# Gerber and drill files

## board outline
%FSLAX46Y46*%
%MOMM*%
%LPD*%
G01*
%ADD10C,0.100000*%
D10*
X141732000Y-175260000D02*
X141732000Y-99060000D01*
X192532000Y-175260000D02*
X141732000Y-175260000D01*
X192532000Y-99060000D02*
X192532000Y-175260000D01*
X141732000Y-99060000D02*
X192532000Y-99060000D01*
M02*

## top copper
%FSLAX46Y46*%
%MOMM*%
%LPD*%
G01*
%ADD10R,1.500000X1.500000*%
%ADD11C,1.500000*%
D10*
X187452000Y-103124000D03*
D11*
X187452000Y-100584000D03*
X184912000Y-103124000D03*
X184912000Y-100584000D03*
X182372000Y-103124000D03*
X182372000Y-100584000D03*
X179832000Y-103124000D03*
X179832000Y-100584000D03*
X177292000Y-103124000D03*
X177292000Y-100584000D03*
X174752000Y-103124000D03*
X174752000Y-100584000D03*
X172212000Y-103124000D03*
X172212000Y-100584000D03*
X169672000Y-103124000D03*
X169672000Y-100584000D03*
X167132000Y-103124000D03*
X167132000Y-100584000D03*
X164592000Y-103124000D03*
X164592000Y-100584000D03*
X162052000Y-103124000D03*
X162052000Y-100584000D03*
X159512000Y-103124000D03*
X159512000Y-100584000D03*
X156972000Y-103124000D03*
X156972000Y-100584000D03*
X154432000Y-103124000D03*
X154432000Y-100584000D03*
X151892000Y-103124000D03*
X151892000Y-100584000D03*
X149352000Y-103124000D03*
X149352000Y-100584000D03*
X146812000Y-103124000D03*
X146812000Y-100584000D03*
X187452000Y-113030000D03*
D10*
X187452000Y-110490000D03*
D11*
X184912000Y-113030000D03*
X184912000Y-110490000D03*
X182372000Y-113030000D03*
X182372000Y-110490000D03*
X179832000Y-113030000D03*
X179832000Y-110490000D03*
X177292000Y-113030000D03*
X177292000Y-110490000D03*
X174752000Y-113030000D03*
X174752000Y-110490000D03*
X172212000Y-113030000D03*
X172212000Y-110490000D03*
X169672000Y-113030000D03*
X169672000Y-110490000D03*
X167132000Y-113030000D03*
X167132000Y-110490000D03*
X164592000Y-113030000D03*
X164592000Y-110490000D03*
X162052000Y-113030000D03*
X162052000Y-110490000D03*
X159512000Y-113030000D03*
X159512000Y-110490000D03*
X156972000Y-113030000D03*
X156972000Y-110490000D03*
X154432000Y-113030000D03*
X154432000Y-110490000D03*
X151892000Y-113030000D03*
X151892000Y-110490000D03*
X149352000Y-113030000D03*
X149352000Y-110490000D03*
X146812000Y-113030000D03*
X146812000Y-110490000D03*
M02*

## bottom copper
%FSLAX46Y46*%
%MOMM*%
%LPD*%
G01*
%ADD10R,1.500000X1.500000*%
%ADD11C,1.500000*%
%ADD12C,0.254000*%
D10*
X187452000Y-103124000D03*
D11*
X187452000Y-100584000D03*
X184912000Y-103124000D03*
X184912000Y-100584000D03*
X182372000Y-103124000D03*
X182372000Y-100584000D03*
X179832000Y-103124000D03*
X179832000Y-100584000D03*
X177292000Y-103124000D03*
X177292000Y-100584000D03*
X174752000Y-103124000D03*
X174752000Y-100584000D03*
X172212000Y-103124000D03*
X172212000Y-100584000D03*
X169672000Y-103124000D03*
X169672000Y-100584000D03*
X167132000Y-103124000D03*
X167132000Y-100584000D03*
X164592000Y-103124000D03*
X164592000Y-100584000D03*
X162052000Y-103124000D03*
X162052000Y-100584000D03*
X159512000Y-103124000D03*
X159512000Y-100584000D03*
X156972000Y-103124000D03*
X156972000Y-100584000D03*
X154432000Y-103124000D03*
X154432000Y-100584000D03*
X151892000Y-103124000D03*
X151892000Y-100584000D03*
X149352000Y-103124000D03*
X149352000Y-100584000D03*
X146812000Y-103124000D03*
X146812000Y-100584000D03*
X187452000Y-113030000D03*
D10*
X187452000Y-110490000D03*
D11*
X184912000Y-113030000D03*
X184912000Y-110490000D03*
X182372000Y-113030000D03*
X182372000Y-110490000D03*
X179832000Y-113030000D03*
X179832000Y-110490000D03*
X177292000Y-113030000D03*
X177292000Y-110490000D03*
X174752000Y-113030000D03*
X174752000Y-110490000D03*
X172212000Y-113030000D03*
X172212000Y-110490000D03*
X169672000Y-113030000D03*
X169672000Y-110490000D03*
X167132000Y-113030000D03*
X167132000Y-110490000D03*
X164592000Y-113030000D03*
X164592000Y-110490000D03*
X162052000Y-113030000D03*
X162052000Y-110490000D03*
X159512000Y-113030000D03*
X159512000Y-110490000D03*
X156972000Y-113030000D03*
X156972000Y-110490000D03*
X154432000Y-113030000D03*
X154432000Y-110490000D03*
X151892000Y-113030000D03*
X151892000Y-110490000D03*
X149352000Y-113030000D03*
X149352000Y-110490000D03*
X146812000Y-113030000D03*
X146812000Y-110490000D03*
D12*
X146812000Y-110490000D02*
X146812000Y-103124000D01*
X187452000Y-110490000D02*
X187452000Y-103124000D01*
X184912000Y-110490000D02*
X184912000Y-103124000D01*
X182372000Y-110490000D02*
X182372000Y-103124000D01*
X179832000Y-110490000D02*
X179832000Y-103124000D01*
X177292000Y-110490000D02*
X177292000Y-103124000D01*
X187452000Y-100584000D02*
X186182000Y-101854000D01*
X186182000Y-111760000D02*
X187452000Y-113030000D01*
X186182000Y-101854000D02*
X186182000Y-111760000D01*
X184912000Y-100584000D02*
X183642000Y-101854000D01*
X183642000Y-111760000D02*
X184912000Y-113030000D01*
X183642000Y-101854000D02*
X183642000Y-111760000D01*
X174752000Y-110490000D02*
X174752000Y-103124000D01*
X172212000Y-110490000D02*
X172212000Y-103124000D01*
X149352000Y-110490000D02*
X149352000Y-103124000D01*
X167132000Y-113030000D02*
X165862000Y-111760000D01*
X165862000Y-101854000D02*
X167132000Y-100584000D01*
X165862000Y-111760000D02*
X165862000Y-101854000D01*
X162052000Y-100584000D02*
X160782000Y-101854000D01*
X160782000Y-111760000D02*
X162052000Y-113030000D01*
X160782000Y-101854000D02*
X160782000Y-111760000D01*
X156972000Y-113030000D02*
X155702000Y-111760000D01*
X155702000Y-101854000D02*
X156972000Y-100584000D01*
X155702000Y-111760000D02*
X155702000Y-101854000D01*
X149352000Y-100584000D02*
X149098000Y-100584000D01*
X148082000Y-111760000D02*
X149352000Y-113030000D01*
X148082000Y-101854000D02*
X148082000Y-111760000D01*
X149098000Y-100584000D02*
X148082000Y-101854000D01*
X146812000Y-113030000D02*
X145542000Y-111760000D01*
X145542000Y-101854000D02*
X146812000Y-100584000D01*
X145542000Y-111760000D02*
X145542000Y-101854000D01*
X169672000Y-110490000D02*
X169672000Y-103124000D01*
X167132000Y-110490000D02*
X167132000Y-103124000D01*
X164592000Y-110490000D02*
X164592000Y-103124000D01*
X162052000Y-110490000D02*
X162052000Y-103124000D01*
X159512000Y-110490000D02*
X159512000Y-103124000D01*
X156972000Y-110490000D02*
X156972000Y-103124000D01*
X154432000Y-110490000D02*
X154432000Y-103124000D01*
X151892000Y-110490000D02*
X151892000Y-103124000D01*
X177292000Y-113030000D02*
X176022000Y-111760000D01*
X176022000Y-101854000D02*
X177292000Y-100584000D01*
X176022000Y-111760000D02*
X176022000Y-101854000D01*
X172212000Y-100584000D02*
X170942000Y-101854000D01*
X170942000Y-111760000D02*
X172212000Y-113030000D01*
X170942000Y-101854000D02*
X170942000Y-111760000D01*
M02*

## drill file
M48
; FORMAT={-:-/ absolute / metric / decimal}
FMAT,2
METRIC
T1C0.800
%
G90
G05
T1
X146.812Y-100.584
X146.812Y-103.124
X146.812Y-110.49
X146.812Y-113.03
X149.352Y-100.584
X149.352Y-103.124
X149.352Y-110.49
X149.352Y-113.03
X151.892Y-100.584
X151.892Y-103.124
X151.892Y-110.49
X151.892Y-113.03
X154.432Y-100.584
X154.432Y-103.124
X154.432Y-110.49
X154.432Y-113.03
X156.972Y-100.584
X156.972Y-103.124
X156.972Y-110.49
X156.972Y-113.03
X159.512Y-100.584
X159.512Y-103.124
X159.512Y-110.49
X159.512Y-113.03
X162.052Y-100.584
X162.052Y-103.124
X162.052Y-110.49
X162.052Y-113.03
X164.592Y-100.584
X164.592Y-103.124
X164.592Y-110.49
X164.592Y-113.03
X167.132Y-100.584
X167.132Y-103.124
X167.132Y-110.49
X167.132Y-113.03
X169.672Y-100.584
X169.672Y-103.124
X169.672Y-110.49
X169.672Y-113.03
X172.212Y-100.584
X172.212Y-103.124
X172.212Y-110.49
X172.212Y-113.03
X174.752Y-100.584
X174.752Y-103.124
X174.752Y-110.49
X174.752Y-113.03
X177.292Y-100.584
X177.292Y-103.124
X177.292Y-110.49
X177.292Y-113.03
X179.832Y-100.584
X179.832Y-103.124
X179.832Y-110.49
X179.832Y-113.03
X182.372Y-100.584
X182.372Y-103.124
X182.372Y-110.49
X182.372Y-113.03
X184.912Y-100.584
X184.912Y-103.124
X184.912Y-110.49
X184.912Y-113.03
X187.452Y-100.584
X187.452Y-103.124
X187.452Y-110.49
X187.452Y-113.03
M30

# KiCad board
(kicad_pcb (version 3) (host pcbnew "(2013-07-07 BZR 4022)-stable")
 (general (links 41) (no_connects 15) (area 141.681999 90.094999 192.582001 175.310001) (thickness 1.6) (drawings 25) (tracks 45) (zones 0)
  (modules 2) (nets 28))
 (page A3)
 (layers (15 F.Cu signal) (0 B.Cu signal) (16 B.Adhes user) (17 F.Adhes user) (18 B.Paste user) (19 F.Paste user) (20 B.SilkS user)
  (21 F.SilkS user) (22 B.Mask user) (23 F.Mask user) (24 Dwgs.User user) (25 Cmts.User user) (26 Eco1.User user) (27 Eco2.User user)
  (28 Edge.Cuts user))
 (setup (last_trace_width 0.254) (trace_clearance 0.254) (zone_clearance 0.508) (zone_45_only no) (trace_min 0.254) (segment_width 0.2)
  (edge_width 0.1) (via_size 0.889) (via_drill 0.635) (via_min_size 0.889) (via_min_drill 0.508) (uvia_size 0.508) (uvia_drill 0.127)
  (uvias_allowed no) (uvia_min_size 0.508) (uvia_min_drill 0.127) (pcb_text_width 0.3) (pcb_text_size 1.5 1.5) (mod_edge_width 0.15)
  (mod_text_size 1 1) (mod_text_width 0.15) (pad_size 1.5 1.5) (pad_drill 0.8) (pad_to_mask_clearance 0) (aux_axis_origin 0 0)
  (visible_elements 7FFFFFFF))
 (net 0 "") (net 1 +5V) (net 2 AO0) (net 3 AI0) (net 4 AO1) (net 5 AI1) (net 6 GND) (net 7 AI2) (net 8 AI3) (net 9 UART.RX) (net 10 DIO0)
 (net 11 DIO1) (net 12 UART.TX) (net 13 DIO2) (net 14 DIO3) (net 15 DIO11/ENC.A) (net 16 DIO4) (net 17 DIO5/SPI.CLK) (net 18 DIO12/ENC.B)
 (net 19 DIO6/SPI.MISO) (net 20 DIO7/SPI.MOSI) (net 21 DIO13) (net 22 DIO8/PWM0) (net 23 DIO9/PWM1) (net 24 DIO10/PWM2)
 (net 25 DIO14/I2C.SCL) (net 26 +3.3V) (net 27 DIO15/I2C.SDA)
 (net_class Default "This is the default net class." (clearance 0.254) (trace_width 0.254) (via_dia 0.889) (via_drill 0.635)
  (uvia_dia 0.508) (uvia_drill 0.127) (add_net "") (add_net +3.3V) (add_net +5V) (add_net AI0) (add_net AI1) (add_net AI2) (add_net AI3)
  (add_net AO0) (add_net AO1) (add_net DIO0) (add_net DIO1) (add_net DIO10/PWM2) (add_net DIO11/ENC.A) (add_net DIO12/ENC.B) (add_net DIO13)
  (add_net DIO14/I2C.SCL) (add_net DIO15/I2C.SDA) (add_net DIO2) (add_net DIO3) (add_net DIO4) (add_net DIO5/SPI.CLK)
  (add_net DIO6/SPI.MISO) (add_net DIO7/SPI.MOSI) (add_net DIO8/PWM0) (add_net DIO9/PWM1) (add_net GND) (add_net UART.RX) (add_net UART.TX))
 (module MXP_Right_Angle (layer F.Cu) (at 168.402 101.854)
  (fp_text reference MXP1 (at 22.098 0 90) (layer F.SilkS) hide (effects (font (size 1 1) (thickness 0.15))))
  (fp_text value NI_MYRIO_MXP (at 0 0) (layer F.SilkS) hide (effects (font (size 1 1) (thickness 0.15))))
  (pad 1 thru_hole rect (at 19.05 1.27) (size 1.5 1.5) (drill 0.8) (layers *.Cu *.Mask F.SilkS) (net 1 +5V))
  (pad 2 thru_hole circle (at 19.05 -1.27) (size 1.5 1.5) (drill 0.8) (layers *.Cu *.Mask F.SilkS) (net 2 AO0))
  (pad 3 thru_hole circle (at 16.51 1.27) (size 1.5 1.5) (drill 0.8) (layers *.Cu *.Mask F.SilkS) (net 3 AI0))
  (pad 4 thru_hole circle (at 16.51 -1.27) (size 1.5 1.5) (drill 0.8) (layers *.Cu *.Mask F.SilkS) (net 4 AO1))
  (pad 5 thru_hole circle (at 13.97 1.27) (size 1.5 1.5) (drill 0.8) (layers *.Cu *.Mask F.SilkS) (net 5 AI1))
  (pad 6 thru_hole circle (at 13.97 -1.27) (size 1.5 1.5) (drill 0.8) (layers *.Cu *.Mask F.SilkS) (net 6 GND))
  (pad 7 thru_hole circle (at 11.43 1.27) (size 1.5 1.5) (drill 0.8) (layers *.Cu *.Mask F.SilkS) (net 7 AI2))
  (pad 8 thru_hole circle (at 11.43 -1.27) (size 1.5 1.5) (drill 0.8) (layers *.Cu *.Mask F.SilkS) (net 6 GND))
  (pad 9 thru_hole circle (at 8.89 1.27) (size 1.5 1.5) (drill 0.8) (layers *.Cu *.Mask F.SilkS) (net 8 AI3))
  (pad 10 thru_hole circle (at 8.89 -1.27) (size 1.5 1.5) (drill 0.8) (layers *.Cu *.Mask F.SilkS) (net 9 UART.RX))
  (pad 11 thru_hole circle (at 6.35 1.27) (size 1.5 1.5) (drill 0.8) (layers *.Cu *.Mask F.SilkS) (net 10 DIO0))
  (pad 12 thru_hole circle (at 6.35 -1.27) (size 1.5 1.5) (drill 0.8) (layers *.Cu *.Mask F.SilkS) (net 6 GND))
  (pad 13 thru_hole circle (at 3.81 1.27) (size 1.5 1.5) (drill 0.8) (layers *.Cu *.Mask F.SilkS) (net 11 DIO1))
  (pad 14 thru_hole circle (at 3.81 -1.27) (size 1.5 1.5) (drill 0.8) (layers *.Cu *.Mask F.SilkS) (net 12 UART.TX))
  (pad 15 thru_hole circle (at 1.27 1.27) (size 1.5 1.5) (drill 0.8) (layers *.Cu *.Mask F.SilkS) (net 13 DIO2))
  (pad 16 thru_hole circle (at 1.27 -1.27) (size 1.5 1.5) (drill 0.8) (layers *.Cu *.Mask F.SilkS) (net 6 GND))
  (pad 17 thru_hole circle (at -1.27 1.27) (size 1.5 1.5) (drill 0.8) (layers *.Cu *.Mask F.SilkS) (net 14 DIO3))
  (pad 18 thru_hole circle (at -1.27 -1.27) (size 1.5 1.5) (drill 0.8) (layers *.Cu *.Mask F.SilkS) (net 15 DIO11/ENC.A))
  (pad 19 thru_hole circle (at -3.81 1.27) (size 1.5 1.5) (drill 0.8) (layers *.Cu *.Mask F.SilkS) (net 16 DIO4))
  (pad 20 thru_hole circle (at -3.81 -1.27) (size 1.5 1.5) (drill 0.8) (layers *.Cu *.Mask F.SilkS) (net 6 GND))
  (pad 21 thru_hole circle (at -6.35 1.27) (size 1.5 1.5) (drill 0.8) (layers *.Cu *.Mask F.SilkS) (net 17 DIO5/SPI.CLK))
  (pad 22 thru_hole circle (at -6.35 -1.27) (size 1.5 1.5) (drill 0.8) (layers *.Cu *.Mask F.SilkS) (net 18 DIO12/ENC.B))
  (pad 23 thru_hole circle (at -8.89 1.27) (size 1.5 1.5) (drill 0.8) (layers *.Cu *.Mask F.SilkS) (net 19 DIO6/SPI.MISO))
  (pad 24 thru_hole circle (at -8.89 -1.27) (size 1.5 1.5) (drill 0.8) (layers *.Cu *.Mask F.SilkS) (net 6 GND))
  (pad 25 thru_hole circle (at -11.43 1.27) (size 1.5 1.5) (drill 0.8) (layers *.Cu *.Mask F.SilkS) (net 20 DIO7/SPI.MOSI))
  (pad 26 thru_hole circle (at -11.43 -1.27) (size 1.5 1.5) (drill 0.8) (layers *.Cu *.Mask F.SilkS) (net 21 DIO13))
  (pad 27 thru_hole circle (at -13.97 1.27) (size 1.5 1.5) (drill 0.8) (layers *.Cu *.Mask F.SilkS) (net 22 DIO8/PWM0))
  (pad 28 thru_hole circle (at -13.97 -1.27) (size 1.5 1.5) (drill 0.8) (layers *.Cu *.Mask F.SilkS) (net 6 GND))
  (pad 29 thru_hole circle (at -16.51 1.27) (size 1.5 1.5) (drill 0.8) (layers *.Cu *.Mask F.SilkS) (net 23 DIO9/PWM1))
  (pad 30 thru_hole circle (at -16.51 -1.27) (size 1.5 1.5) (drill 0.8) (layers *.Cu *.Mask F.SilkS) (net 6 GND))
  (pad 31 thru_hole circle (at -19.05 1.27) (size 1.5 1.5) (drill 0.8) (layers *.Cu *.Mask F.SilkS) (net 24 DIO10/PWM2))
  (pad 32 thru_hole circle (at -19.05 -1.27) (size 1.5 1.5) (drill 0.8) (layers *.Cu *.Mask F.SilkS) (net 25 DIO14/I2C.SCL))
  (pad 33 thru_hole circle (at -21.59 1.27) (size 1.5 1.5) (drill 0.8) (layers *.Cu *.Mask F.SilkS) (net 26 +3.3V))
  (pad 34 thru_hole circle (at -21.59 -1.27) (size 1.5 1.5) (drill 0.8) (layers *.Cu *.Mask F.SilkS) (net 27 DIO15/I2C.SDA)))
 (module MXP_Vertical (layer F.Cu) (at 168.402 111.76)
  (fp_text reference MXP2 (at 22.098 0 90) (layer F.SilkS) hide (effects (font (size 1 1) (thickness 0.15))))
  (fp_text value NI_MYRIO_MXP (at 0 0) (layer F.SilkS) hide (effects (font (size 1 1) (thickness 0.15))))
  (pad 2 thru_hole circle (at 19.05 1.27) (size 1.5 1.5) (drill 0.8) (layers *.Cu *.Mask F.SilkS) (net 2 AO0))
  (pad 1 thru_hole rect (at 19.05 -1.27) (size 1.5 1.5) (drill 0.8) (layers *.Cu *.Mask F.SilkS) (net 1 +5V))
  (pad 4 thru_hole circle (at 16.51 1.27) (size 1.5 1.5) (drill 0.8) (layers *.Cu *.Mask F.SilkS) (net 4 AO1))
  (pad 3 thru_hole circle (at 16.51 -1.27) (size 1.5 1.5) (drill 0.8) (layers *.Cu *.Mask F.SilkS) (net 3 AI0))
  (pad 6 thru_hole circle (at 13.97 1.27) (size 1.5 1.5) (drill 0.8) (layers *.Cu *.Mask F.SilkS) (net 6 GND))
  (pad 5 thru_hole circle (at 13.97 -1.27) (size 1.5 1.5) (drill 0.8) (layers *.Cu *.Mask F.SilkS) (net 5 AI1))
  (pad 8 thru_hole circle (at 11.43 1.27) (size 1.5 1.5) (drill 0.8) (layers *.Cu *.Mask F.SilkS) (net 6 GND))
  (pad 7 thru_hole circle (at 11.43 -1.27) (size 1.5 1.5) (drill 0.8) (layers *.Cu *.Mask F.SilkS) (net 7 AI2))
  (pad 10 thru_hole circle (at 8.89 1.27) (size 1.5 1.5) (drill 0.8) (layers *.Cu *.Mask F.SilkS) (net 9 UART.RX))
  (pad 9 thru_hole circle (at 8.89 -1.27) (size 1.5 1.5) (drill 0.8) (layers *.Cu *.Mask F.SilkS) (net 8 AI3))
  (pad 12 thru_hole circle (at 6.35 1.27) (size 1.5 1.5) (drill 0.8) (layers *.Cu *.Mask F.SilkS) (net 6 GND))
  (pad 11 thru_hole circle (at 6.35 -1.27) (size 1.5 1.5) (drill 0.8) (layers *.Cu *.Mask F.SilkS) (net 10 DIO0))
  (pad 14 thru_hole circle (at 3.81 1.27) (size 1.5 1.5) (drill 0.8) (layers *.Cu *.Mask F.SilkS) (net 12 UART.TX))
  (pad 13 thru_hole circle (at 3.81 -1.27) (size 1.5 1.5) (drill 0.8) (layers *.Cu *.Mask F.SilkS) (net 11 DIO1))
  (pad 16 thru_hole circle (at 1.27 1.27) (size 1.5 1.5) (drill 0.8) (layers *.Cu *.Mask F.SilkS) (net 6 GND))
  (pad 15 thru_hole circle (at 1.27 -1.27) (size 1.5 1.5) (drill 0.8) (layers *.Cu *.Mask F.SilkS) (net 13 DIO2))
  (pad 18 thru_hole circle (at -1.27 1.27) (size 1.5 1.5) (drill 0.8) (layers *.Cu *.Mask F.SilkS) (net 15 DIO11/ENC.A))
  (pad 17 thru_hole circle (at -1.27 -1.27) (size 1.5 1.5) (drill 0.8) (layers *.Cu *.Mask F.SilkS) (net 14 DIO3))
  (pad 20 thru_hole circle (at -3.81 1.27) (size 1.5 1.5) (drill 0.8) (layers *.Cu *.Mask F.SilkS) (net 6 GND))
  (pad 19 thru_hole circle (at -3.81 -1.27) (size 1.5 1.5) (drill 0.8) (layers *.Cu *.Mask F.SilkS) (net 16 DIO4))
  (pad 22 thru_hole circle (at -6.35 1.27) (size 1.5 1.5) (drill 0.8) (layers *.Cu *.Mask F.SilkS) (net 18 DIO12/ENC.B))
  (pad 21 thru_hole circle (at -6.35 -1.27) (size 1.5 1.5) (drill 0.8) (layers *.Cu *.Mask F.SilkS) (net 17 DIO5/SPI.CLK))
  (pad 24 thru_hole circle (at -8.89 1.27) (size 1.5 1.5) (drill 0.8) (layers *.Cu *.Mask F.SilkS) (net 6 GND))
  (pad 23 thru_hole circle (at -8.89 -1.27) (size 1.5 1.5) (drill 0.8) (layers *.Cu *.Mask F.SilkS) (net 19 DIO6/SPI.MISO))
  (pad 26 thru_hole circle (at -11.43 1.27) (size 1.5 1.5) (drill 0.8) (layers *.Cu *.Mask F.SilkS) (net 21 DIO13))
  (pad 25 thru_hole circle (at -11.43 -1.27) (size 1.5 1.5) (drill 0.8) (layers *.Cu *.Mask F.SilkS) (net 20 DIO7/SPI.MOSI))
  (pad 28 thru_hole circle (at -13.97 1.27) (size 1.5 1.5) (drill 0.8) (layers *.Cu *.Mask F.SilkS) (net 6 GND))
  (pad 27 thru_hole circle (at -13.97 -1.27) (size 1.5 1.5) (drill 0.8) (layers *.Cu *.Mask F.SilkS) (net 22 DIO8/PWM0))
  (pad 30 thru_hole circle (at -16.51 1.27) (size 1.5 1.5) (drill 0.8) (layers *.Cu *.Mask F.SilkS) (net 6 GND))
  (pad 29 thru_hole circle (at -16.51 -1.27) (size 1.5 1.5) (drill 0.8) (layers *.Cu *.Mask F.SilkS) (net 23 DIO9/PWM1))
  (pad 32 thru_hole circle (at -19.05 1.27) (size 1.5 1.5) (drill 0.8) (layers *.Cu *.Mask F.SilkS) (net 25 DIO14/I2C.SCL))
  (pad 31 thru_hole circle (at -19.05 -1.27) (size 1.5 1.5) (drill 0.8) (layers *.Cu *.Mask F.SilkS) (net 24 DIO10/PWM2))
  (pad 34 thru_hole circle (at -21.59 1.27) (size 1.5 1.5) (drill 0.8) (layers *.Cu *.Mask F.SilkS) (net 27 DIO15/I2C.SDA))
  (pad 33 thru_hole circle (at -21.59 -1.27) (size 1.5 1.5) (drill 0.8) (layers *.Cu *.Mask F.SilkS) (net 26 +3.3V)))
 (gr_line (start 141.732 175.26) (end 141.732 99.06) (angle 90) (layer Edge.Cuts) (width 0.1))
 (gr_line (start 192.532 175.26) (end 141.732 175.26) (angle 90) (layer Edge.Cuts) (width 0.1))
 (gr_line (start 192.532 99.06) (end 192.532 175.26) (angle 90) (layer Edge.Cuts) (width 0.1))
 (gr_line (start 141.732 99.06) (end 192.532 99.06) (angle 90) (layer Edge.Cuts) (width 0.1))
 (segment (start 146.812 110.49) (end 146.812 103.124) (width 0.254) (layer B.Cu) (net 26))
 (segment (start 187.452 110.49) (end 187.452 103.124) (width 0.254) (layer B.Cu) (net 1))
 (segment (start 184.912 110.49) (end 184.912 103.124) (width 0.254) (layer B.Cu) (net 3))
 (segment (start 182.372 110.49) (end 182.372 103.124) (width 0.254) (layer B.Cu) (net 5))
 (segment (start 179.832 110.49) (end 179.832 103.124) (width 0.254) (layer B.Cu) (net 7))
 (segment (start 177.292 110.49) (end 177.292 103.124) (width 0.254) (layer B.Cu) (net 8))
 (segment (start 187.452 100.584) (end 186.182 101.854) (width 0.254) (layer B.Cu) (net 2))
 (segment (start 186.182 111.76) (end 187.452 113.03) (width 0.254) (layer B.Cu) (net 2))
 (segment (start 186.182 101.854) (end 186.182 111.76) (width 0.254) (layer B.Cu) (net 2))
 (segment (start 184.912 100.584) (end 183.642 101.854) (width 0.254) (layer B.Cu) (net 4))
 (segment (start 183.642 111.76) (end 184.912 113.03) (width 0.254) (layer B.Cu) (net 4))
 (segment (start 183.642 101.854) (end 183.642 111.76) (width 0.254) (layer B.Cu) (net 4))
 (segment (start 174.752 110.49) (end 174.752 103.124) (width 0.254) (layer B.Cu) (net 10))
 (segment (start 172.212 110.49) (end 172.212 103.124) (width 0.254) (layer B.Cu) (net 11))
 (segment (start 149.352 110.49) (end 149.352 103.124) (width 0.254) (layer B.Cu) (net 24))
 (segment (start 167.132 113.03) (end 165.862 111.76) (width 0.254) (layer B.Cu) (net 15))
 (segment (start 165.862 101.854) (end 167.132 100.584) (width 0.254) (layer B.Cu) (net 15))
 (segment (start 165.862 111.76) (end 165.862 101.854) (width 0.254) (layer B.Cu) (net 15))
 (segment (start 162.052 100.584) (end 160.782 101.854) (width 0.254) (layer B.Cu) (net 18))
 (segment (start 160.782 111.76) (end 162.052 113.03) (width 0.254) (layer B.Cu) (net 18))
 (segment (start 160.782 101.854) (end 160.782 111.76) (width 0.254) (layer B.Cu) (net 18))
 (segment (start 156.972 113.03) (end 155.702 111.76) (width 0.254) (layer B.Cu) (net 21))
 (segment (start 155.702 101.854) (end 156.972 100.584) (width 0.254) (layer B.Cu) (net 21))
 (segment (start 155.702 111.76) (end 155.702 101.854) (width 0.254) (layer B.Cu) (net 21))
 (segment (start 149.352 100.584) (end 149.098 100.584) (width 0.254) (layer B.Cu) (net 25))
 (segment (start 148.082 111.76) (end 149.352 113.03) (width 0.254) (layer B.Cu) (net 25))
 (segment (start 148.082 101.854) (end 148.082 111.76) (width 0.254) (layer B.Cu) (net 25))
 (segment (start 149.098 100.584) (end 148.082 101.854) (width 0.254) (layer B.Cu) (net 25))
 (segment (start 146.812 113.03) (end 145.542 111.76) (width 0.254) (layer B.Cu) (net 27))
 (segment (start 145.542 101.854) (end 146.812 100.584) (width 0.254) (layer B.Cu) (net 27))
 (segment (start 145.542 111.76) (end 145.542 101.854) (width 0.254) (layer B.Cu) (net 27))
 (segment (start 169.672 110.49) (end 169.672 103.124) (width 0.254) (layer B.Cu) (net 13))
 (segment (start 167.132 110.49) (end 167.132 103.124) (width 0.254) (layer B.Cu) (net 14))
 (segment (start 164.592 110.49) (end 164.592 103.124) (width 0.254) (layer B.Cu) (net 16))
 (segment (start 162.052 110.49) (end 162.052 103.124) (width 0.254) (layer B.Cu) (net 17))
 (segment (start 159.512 110.49) (end 159.512 103.124) (width 0.254) (layer B.Cu) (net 19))
 (segment (start 156.972 110.49) (end 156.972 103.124) (width 0.254) (layer B.Cu) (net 20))
 (segment (start 154.432 110.49) (end 154.432 103.124) (width 0.254) (layer B.Cu) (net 22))
 (segment (start 151.892 110.49) (end 151.892 103.124) (width 0.254) (layer B.Cu) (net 23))
 (segment (start 177.292 113.03) (end 176.022 111.76) (width 0.254) (layer B.Cu) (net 9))
 (segment (start 176.022 101.854) (end 177.292 100.584) (width 0.254) (layer B.Cu) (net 9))
 (segment (start 176.022 111.76) (end 176.022 101.854) (width 0.254) (layer B.Cu) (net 9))
 (segment (start 172.212 100.584) (end 170.942 101.854) (width 0.254) (layer B.Cu) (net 12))
 (segment (start 170.942 111.76) (end 172.212 113.03) (width 0.254) (layer B.Cu) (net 12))
 (segment (start 170.942 101.854) (end 170.942 111.76) (width 0.254) (layer B.Cu) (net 12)))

